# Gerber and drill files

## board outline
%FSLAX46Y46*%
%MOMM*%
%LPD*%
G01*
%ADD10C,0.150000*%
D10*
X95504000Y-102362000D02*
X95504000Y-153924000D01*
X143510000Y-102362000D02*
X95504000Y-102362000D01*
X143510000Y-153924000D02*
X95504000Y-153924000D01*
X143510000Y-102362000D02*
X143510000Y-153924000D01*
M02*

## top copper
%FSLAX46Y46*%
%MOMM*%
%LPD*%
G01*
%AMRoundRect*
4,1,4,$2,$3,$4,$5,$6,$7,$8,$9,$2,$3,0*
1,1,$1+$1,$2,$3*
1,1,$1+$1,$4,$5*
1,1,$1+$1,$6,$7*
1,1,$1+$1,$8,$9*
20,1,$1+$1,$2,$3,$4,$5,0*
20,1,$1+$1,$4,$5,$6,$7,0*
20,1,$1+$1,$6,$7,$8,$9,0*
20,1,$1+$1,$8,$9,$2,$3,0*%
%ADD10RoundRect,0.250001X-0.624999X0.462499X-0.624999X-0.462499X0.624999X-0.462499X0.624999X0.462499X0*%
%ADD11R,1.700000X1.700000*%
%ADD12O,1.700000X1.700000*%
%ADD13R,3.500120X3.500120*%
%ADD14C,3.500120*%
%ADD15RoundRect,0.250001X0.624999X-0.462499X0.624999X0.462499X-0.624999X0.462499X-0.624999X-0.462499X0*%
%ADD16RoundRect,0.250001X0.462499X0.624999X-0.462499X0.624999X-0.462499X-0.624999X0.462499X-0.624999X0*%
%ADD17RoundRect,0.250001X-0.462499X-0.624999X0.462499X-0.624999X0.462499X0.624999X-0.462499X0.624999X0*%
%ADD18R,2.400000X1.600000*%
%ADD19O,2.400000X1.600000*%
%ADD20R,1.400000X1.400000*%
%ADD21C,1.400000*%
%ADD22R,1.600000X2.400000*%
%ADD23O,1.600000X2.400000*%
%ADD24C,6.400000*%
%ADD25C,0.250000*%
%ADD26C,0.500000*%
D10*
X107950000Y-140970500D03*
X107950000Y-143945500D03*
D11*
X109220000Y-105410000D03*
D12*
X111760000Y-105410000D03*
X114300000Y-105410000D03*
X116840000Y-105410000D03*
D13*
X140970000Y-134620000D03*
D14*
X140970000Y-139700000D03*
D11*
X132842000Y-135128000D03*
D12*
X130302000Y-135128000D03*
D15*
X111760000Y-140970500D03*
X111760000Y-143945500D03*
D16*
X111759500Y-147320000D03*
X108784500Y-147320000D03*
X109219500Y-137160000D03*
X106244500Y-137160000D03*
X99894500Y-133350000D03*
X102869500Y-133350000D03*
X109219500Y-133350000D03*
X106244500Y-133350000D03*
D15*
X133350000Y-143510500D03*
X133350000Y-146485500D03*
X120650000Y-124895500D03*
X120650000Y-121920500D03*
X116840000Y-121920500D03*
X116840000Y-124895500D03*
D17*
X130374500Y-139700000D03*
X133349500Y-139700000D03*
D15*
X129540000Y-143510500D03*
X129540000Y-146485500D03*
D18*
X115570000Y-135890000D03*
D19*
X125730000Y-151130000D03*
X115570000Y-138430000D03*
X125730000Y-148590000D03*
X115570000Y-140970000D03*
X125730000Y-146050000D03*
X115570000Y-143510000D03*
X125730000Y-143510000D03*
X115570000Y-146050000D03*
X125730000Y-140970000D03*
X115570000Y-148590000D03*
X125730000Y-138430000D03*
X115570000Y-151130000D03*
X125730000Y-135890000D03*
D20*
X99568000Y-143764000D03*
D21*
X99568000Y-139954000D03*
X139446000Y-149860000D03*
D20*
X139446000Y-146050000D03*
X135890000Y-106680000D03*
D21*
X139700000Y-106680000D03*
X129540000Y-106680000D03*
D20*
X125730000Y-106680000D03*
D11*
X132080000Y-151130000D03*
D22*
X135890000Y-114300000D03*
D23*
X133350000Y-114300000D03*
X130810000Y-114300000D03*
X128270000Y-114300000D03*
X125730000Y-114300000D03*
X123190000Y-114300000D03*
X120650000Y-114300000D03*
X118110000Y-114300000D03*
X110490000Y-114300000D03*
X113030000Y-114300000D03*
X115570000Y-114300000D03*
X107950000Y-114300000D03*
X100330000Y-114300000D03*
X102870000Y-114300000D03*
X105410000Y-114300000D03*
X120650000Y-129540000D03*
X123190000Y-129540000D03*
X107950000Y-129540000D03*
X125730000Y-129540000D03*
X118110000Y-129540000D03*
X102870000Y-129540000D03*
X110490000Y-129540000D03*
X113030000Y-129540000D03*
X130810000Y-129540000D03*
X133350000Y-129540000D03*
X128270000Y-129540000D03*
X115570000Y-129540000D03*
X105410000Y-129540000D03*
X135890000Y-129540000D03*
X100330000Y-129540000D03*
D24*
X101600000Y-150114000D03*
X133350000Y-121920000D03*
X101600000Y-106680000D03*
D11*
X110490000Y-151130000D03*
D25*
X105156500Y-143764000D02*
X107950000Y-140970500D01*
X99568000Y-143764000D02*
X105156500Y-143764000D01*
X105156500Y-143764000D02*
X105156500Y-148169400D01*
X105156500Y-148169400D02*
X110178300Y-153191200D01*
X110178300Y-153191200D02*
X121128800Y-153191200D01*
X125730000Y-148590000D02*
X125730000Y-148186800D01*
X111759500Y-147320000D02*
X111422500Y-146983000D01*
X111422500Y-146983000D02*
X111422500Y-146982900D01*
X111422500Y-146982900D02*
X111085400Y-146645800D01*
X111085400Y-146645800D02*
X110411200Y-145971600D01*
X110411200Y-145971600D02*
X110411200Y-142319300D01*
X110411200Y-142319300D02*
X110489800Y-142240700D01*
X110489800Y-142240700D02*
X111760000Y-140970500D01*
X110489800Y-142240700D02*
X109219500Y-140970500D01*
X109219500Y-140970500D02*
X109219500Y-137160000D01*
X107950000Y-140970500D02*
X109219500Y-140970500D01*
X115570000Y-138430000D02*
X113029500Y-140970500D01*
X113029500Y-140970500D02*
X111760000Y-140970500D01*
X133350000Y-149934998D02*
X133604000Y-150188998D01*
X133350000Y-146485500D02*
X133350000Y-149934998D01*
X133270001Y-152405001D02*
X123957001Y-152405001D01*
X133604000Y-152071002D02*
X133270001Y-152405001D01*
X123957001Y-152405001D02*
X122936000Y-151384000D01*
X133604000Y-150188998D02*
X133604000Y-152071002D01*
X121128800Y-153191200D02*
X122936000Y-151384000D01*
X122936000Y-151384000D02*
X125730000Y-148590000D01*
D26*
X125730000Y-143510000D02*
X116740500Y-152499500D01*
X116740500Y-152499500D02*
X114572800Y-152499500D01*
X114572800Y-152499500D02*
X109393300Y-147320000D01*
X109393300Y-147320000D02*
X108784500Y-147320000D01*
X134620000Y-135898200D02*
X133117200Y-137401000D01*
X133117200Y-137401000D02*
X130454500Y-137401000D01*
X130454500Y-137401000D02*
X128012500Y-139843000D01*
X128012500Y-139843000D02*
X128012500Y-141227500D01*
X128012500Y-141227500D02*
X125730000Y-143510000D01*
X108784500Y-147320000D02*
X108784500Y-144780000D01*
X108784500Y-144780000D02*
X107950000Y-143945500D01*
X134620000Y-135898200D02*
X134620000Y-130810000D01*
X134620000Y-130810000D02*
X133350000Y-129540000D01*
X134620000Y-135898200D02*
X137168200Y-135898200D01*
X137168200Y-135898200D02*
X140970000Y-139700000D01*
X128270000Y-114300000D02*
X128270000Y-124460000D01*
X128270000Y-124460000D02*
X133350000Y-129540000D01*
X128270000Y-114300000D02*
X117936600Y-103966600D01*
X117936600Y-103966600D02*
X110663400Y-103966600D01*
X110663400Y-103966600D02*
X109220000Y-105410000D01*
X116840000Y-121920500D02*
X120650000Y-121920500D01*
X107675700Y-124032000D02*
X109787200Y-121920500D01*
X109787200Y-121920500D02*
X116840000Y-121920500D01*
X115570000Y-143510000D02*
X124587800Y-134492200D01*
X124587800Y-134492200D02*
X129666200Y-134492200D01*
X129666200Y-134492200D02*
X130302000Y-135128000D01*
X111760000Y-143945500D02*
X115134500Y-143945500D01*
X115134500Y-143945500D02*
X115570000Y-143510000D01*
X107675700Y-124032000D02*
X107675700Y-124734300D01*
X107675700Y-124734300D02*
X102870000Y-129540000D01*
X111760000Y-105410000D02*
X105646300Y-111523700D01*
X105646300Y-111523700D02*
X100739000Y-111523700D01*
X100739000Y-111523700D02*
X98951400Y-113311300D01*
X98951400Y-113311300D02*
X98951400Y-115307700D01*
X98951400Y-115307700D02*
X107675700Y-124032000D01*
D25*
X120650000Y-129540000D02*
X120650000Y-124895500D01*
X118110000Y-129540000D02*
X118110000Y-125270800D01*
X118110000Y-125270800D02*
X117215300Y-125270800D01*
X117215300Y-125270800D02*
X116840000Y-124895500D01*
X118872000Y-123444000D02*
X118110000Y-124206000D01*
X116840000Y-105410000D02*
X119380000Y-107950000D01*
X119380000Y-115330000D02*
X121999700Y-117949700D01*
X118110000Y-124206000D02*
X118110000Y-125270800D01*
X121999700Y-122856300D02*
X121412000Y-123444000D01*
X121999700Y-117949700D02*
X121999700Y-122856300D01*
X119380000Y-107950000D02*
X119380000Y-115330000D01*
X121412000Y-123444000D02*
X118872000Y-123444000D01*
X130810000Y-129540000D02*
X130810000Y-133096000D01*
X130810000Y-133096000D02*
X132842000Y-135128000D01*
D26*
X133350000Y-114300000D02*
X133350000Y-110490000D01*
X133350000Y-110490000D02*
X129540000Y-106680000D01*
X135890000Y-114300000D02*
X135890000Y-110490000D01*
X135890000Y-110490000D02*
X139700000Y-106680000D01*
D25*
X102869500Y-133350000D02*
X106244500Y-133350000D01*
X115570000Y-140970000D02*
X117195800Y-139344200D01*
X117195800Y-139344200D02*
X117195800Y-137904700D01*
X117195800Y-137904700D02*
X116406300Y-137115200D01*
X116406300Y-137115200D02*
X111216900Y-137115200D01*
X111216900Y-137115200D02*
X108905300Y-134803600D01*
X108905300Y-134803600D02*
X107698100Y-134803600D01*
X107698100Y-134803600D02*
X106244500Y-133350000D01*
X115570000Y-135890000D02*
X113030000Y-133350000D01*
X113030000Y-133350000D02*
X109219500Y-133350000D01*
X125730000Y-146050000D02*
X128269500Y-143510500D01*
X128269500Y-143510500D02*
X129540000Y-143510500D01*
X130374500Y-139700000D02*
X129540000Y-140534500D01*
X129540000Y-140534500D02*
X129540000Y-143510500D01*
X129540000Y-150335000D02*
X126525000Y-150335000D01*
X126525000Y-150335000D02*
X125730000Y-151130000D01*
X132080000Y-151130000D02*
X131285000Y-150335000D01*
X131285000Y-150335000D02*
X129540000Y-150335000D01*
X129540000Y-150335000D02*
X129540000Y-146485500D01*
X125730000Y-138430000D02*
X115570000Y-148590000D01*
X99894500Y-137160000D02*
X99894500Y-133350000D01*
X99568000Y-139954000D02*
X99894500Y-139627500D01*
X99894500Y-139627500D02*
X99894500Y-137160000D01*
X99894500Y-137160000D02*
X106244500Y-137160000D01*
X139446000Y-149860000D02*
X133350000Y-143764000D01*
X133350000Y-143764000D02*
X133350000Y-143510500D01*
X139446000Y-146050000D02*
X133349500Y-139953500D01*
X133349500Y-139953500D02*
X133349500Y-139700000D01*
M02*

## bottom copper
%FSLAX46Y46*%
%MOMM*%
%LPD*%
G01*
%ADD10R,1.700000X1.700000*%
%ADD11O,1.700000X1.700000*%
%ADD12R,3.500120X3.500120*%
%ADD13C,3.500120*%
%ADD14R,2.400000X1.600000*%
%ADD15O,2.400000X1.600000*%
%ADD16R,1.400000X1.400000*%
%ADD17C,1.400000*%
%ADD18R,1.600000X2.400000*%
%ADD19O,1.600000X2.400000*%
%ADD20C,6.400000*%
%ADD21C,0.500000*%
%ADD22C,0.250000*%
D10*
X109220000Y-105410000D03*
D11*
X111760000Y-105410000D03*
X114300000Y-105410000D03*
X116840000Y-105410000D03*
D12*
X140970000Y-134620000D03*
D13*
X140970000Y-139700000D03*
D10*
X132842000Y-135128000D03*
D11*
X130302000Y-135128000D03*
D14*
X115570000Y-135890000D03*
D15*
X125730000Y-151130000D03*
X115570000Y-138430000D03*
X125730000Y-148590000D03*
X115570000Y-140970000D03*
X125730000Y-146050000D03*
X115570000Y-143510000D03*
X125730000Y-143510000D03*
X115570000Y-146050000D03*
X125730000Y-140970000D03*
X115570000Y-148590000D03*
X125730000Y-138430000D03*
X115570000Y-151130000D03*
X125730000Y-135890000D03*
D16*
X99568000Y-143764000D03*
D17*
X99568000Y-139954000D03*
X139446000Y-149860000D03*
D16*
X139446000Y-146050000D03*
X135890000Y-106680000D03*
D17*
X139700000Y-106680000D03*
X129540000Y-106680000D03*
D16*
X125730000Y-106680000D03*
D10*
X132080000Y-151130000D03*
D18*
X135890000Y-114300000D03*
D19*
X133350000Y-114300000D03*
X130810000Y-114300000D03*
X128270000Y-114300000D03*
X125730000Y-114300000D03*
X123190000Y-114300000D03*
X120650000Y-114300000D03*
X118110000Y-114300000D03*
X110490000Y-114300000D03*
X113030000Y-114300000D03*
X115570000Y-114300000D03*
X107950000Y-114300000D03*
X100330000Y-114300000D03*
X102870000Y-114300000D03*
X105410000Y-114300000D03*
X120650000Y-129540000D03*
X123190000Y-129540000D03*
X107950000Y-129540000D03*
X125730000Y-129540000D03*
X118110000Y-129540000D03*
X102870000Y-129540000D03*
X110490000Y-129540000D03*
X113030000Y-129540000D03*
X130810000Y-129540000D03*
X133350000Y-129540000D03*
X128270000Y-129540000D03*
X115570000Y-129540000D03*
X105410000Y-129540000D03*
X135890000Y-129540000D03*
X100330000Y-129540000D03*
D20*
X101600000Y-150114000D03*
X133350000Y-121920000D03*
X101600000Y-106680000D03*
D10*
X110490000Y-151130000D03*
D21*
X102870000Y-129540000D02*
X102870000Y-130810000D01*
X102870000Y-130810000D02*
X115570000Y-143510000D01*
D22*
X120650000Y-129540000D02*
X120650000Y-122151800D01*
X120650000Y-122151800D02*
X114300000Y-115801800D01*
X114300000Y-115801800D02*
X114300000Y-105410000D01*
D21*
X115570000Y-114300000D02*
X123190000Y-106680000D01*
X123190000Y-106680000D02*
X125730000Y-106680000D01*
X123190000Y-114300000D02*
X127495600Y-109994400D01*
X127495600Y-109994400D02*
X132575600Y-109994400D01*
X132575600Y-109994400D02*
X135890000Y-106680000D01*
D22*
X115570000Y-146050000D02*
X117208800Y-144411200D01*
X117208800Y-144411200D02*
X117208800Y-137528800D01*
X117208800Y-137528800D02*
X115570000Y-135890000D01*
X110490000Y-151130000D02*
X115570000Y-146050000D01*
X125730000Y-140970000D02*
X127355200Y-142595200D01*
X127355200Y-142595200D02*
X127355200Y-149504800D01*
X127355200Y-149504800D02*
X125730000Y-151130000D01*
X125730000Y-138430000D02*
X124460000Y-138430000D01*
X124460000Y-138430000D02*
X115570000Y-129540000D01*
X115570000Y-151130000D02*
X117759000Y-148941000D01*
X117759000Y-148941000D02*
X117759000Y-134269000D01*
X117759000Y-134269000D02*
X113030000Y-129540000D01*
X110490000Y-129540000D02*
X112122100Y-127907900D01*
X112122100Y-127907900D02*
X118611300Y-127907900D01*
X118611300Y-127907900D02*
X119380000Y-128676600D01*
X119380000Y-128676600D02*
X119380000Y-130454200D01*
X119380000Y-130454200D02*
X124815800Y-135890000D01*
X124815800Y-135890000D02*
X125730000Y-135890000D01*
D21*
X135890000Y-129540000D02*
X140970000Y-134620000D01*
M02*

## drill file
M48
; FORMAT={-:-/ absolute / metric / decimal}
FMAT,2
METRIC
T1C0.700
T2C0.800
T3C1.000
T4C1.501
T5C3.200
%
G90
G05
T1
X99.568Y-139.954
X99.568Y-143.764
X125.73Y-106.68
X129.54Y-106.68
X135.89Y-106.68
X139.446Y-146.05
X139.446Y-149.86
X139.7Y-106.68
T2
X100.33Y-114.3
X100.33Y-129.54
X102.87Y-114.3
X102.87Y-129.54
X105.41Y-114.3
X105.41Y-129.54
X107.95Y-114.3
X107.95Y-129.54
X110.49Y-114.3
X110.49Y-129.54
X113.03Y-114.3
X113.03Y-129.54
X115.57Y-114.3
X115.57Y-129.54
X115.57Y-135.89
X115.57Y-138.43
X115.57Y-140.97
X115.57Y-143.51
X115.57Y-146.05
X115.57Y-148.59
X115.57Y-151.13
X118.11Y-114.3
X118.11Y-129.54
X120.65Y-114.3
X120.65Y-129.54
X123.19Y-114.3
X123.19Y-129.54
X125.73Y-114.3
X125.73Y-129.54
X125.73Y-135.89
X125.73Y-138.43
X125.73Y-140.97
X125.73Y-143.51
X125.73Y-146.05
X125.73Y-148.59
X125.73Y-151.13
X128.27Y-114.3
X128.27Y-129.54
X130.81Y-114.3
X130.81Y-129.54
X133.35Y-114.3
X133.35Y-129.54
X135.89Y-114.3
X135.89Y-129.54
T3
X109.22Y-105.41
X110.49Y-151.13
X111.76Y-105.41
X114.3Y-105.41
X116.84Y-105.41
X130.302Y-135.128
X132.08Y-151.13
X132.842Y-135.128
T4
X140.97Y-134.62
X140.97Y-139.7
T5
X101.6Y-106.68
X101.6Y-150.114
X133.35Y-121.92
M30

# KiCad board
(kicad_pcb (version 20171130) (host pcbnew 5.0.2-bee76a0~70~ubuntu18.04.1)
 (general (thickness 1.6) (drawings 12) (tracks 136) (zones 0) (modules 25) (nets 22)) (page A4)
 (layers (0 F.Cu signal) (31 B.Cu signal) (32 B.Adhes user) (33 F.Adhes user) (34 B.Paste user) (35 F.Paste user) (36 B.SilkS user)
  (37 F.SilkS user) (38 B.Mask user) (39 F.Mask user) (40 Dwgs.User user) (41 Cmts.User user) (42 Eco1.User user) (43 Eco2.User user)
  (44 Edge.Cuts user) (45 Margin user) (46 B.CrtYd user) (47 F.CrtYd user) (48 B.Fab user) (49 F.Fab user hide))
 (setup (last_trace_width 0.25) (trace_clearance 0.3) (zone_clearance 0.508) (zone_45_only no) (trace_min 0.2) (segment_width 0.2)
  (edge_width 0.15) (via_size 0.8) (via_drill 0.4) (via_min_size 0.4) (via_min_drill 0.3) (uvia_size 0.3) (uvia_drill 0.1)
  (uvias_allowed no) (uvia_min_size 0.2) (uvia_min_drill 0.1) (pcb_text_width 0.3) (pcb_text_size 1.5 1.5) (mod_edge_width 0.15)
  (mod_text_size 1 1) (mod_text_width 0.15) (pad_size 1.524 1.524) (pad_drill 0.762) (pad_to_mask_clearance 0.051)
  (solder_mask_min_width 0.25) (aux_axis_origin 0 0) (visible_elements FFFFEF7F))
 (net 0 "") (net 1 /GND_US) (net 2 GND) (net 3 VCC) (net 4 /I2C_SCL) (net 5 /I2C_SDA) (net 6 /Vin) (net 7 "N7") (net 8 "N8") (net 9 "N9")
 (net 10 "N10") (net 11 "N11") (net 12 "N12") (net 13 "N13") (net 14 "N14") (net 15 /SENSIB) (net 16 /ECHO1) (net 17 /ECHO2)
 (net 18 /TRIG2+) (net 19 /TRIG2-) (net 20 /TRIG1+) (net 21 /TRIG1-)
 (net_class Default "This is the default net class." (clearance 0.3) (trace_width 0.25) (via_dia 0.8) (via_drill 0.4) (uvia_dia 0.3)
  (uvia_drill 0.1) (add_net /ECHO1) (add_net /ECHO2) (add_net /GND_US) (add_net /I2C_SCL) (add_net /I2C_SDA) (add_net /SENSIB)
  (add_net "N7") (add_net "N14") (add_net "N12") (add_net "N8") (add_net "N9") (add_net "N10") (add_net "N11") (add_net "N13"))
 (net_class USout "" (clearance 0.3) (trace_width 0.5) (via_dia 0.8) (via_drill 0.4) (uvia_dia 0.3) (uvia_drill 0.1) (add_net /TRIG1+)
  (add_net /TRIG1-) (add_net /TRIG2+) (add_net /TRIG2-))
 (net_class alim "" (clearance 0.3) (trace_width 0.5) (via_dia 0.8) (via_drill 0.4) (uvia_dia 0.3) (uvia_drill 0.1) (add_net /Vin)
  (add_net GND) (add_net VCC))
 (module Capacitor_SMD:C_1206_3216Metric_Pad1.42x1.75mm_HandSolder (layer F.Cu) (at 107.95 142.458 270)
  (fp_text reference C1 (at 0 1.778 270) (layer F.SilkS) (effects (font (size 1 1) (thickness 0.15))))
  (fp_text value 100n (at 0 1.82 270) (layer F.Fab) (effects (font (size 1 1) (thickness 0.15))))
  (pad 1 smd roundrect (at -1.4875 0 270) (size 1.425 1.75) (layers F.Cu F.Paste F.Mask) (roundrect_rratio 0.175439) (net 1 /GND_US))
  (pad 2 smd roundrect (at 1.4875 0 270) (size 1.425 1.75) (layers F.Cu F.Paste F.Mask) (roundrect_rratio 0.175439) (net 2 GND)))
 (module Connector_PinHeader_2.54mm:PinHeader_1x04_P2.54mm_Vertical (layer F.Cu) (at 109.22 105.41 90)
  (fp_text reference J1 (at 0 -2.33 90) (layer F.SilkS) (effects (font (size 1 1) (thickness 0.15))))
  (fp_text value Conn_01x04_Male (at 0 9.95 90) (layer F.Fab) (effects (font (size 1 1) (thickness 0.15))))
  (pad 1 thru_hole rect (at 0 0 90) (size 1.7 1.7) (drill 1) (layers *.Cu *.Mask) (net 2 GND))
  (pad 2 thru_hole oval (at 0 2.54 90) (size 1.7 1.7) (drill 1) (layers *.Cu *.Mask) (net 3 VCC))
  (pad 3 thru_hole oval (at 0 5.08 90) (size 1.7 1.7) (drill 1) (layers *.Cu *.Mask) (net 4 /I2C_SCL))
  (pad 4 thru_hole oval (at 0 7.62 90) (size 1.7 1.7) (drill 1) (layers *.Cu *.Mask) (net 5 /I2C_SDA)))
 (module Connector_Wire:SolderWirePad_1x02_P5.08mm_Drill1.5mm (layer F.Cu) (at 140.97 134.62 270)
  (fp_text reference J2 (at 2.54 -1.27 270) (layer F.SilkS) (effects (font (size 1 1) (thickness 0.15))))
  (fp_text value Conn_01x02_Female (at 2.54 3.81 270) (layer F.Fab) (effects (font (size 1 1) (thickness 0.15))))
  (pad 1 thru_hole rect (at 0 0 270) (size 3.50012 3.50012) (drill 1.50114) (layers *.Cu *.Mask) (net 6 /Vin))
  (pad 2 thru_hole circle (at 5.08 0 270) (size 3.50012 3.50012) (drill 1.50114) (layers *.Cu *.Mask) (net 2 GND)))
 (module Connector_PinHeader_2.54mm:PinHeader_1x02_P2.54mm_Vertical (layer F.Cu) (at 132.842 135.128 270)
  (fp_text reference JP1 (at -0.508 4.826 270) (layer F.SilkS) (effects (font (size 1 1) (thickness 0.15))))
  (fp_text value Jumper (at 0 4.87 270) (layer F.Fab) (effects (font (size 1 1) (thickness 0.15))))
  (pad 1 thru_hole rect (at 0 0 270) (size 1.7 1.7) (drill 1) (layers *.Cu *.Mask) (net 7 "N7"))
  (pad 2 thru_hole oval (at 0 2.54 270) (size 1.7 1.7) (drill 1) (layers *.Cu *.Mask) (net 3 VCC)))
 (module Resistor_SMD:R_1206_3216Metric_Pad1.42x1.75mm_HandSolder (layer F.Cu) (at 111.76 142.458 90)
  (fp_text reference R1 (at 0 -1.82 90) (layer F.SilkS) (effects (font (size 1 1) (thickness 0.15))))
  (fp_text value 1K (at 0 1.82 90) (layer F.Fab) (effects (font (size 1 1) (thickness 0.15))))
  (pad 2 smd roundrect (at 1.4875 0 90) (size 1.425 1.75) (layers F.Cu F.Paste F.Mask) (roundrect_rratio 0.175439) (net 1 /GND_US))
  (pad 1 smd roundrect (at -1.4875 0 90) (size 1.425 1.75) (layers F.Cu F.Paste F.Mask) (roundrect_rratio 0.175439) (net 3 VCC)))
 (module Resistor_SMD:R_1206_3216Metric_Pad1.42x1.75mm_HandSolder (layer F.Cu) (at 110.272 147.32 180)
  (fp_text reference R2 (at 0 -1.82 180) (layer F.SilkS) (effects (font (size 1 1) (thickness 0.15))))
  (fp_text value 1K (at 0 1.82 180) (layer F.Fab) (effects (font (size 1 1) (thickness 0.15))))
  (pad 1 smd roundrect (at -1.4875 0 180) (size 1.425 1.75) (layers F.Cu F.Paste F.Mask) (roundrect_rratio 0.175439) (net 1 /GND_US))
  (pad 2 smd roundrect (at 1.4875 0 180) (size 1.425 1.75) (layers F.Cu F.Paste F.Mask) (roundrect_rratio 0.175439) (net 2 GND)))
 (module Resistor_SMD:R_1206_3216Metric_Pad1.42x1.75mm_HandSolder (layer F.Cu) (at 107.732 137.16 180)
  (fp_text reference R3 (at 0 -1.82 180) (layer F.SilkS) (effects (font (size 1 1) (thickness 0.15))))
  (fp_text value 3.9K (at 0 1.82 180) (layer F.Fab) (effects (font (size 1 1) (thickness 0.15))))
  (pad 1 smd roundrect (at -1.4875 0 180) (size 1.425 1.75) (layers F.Cu F.Paste F.Mask) (roundrect_rratio 0.175439) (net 1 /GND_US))
  (pad 2 smd roundrect (at 1.4875 0 180) (size 1.425 1.75) (layers F.Cu F.Paste F.Mask) (roundrect_rratio 0.175439) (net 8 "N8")))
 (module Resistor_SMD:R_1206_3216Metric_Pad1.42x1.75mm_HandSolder (layer F.Cu) (at 101.382 133.35 180)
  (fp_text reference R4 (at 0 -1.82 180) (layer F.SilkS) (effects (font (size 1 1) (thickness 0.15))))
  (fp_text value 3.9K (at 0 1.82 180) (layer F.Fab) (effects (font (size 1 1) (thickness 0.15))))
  (pad 2 smd roundrect (at 1.4875 0 180) (size 1.425 1.75) (layers F.Cu F.Paste F.Mask) (roundrect_rratio 0.175439) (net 8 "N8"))
  (pad 1 smd roundrect (at -1.4875 0 180) (size 1.425 1.75) (layers F.Cu F.Paste F.Mask) (roundrect_rratio 0.175439) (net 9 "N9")))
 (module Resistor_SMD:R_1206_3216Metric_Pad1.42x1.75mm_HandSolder (layer F.Cu) (at 107.732 133.35 180)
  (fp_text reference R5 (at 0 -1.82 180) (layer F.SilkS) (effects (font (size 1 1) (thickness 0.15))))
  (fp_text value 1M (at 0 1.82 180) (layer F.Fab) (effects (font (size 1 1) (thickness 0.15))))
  (pad 1 smd roundrect (at -1.4875 0 180) (size 1.425 1.75) (layers F.Cu F.Paste F.Mask) (roundrect_rratio 0.175439) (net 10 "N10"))
  (pad 2 smd roundrect (at 1.4875 0 180) (size 1.425 1.75) (layers F.Cu F.Paste F.Mask) (roundrect_rratio 0.175439) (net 9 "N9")))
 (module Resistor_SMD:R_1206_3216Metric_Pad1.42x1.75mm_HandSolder (layer F.Cu) (at 133.35 144.998 90)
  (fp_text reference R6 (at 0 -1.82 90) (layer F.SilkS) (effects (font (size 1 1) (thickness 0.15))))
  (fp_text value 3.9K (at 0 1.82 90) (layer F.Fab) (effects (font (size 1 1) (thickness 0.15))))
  (pad 2 smd roundrect (at 1.4875 0 90) (size 1.425 1.75) (layers F.Cu F.Paste F.Mask) (roundrect_rratio 0.175439) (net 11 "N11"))
  (pad 1 smd roundrect (at -1.4875 0 90) (size 1.425 1.75) (layers F.Cu F.Paste F.Mask) (roundrect_rratio 0.175439) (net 1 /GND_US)))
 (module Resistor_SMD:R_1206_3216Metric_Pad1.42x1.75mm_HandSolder (layer F.Cu) (at 120.65 123.408 90)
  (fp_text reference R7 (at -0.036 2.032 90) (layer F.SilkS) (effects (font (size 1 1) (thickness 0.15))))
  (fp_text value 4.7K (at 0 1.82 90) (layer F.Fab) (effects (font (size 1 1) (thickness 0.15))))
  (pad 1 smd roundrect (at -1.4875 0 90) (size 1.425 1.75) (layers F.Cu F.Paste F.Mask) (roundrect_rratio 0.175439) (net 4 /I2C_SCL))
  (pad 2 smd roundrect (at 1.4875 0 90) (size 1.425 1.75) (layers F.Cu F.Paste F.Mask) (roundrect_rratio 0.175439) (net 3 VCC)))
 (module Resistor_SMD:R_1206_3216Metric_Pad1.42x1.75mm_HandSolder (layer F.Cu) (at 116.84 123.408 90)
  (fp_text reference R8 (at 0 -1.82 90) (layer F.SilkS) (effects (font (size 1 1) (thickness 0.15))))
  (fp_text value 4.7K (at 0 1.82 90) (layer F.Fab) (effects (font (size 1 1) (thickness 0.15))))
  (pad 2 smd roundrect (at 1.4875 0 90) (size 1.425 1.75) (layers F.Cu F.Paste F.Mask) (roundrect_rratio 0.175439) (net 3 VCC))
  (pad 1 smd roundrect (at -1.4875 0 90) (size 1.425 1.75) (layers F.Cu F.Paste F.Mask) (roundrect_rratio 0.175439) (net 5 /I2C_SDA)))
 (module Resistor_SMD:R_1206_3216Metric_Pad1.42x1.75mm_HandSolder (layer F.Cu) (at 131.862 139.7)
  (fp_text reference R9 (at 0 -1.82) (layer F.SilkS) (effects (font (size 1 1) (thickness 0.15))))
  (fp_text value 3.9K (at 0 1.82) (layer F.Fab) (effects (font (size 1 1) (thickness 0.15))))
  (pad 1 smd roundrect (at -1.4875 0) (size 1.425 1.75) (layers F.Cu F.Paste F.Mask) (roundrect_rratio 0.175439) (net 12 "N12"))
  (pad 2 smd roundrect (at 1.4875 0) (size 1.425 1.75) (layers F.Cu F.Paste F.Mask) (roundrect_rratio 0.175439) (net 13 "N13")))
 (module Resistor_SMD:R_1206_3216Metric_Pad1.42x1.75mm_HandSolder (layer F.Cu) (at 129.54 144.998 90)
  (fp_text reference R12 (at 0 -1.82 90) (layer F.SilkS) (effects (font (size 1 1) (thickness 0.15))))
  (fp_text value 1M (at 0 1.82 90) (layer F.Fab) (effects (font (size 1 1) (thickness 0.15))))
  (pad 2 smd roundrect (at 1.4875 0 90) (size 1.425 1.75) (layers F.Cu F.Paste F.Mask) (roundrect_rratio 0.175439) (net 12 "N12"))
  (pad 1 smd roundrect (at -1.4875 0 90) (size 1.425 1.75) (layers F.Cu F.Paste F.Mask) (roundrect_rratio 0.175439) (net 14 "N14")))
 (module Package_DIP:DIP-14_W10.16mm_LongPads (layer F.Cu) (at 115.57 135.89)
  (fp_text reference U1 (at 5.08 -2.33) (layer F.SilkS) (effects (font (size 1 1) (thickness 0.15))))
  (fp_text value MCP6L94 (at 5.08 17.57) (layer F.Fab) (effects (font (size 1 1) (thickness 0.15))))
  (pad 1 thru_hole rect (at 0 0) (size 2.4 1.6) (drill 0.8) (layers *.Cu *.Mask) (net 10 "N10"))
  (pad 8 thru_hole oval (at 10.16 15.24) (size 2.4 1.6) (drill 0.8) (layers *.Cu *.Mask) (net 14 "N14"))
  (pad 2 thru_hole oval (at 0 2.54) (size 2.4 1.6) (drill 0.8) (layers *.Cu *.Mask) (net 1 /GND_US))
  (pad 9 thru_hole oval (at 10.16 12.7) (size 2.4 1.6) (drill 0.8) (layers *.Cu *.Mask) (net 1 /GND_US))
  (pad 3 thru_hole oval (at 0 5.08) (size 2.4 1.6) (drill 0.8) (layers *.Cu *.Mask) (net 9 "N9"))
  (pad 10 thru_hole oval (at 10.16 10.16) (size 2.4 1.6) (drill 0.8) (layers *.Cu *.Mask) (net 12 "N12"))
  (pad 4 thru_hole oval (at 0 7.62) (size 2.4 1.6) (drill 0.8) (layers *.Cu *.Mask) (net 3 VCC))
  (pad 11 thru_hole oval (at 10.16 7.62) (size 2.4 1.6) (drill 0.8) (layers *.Cu *.Mask) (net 2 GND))
  (pad 5 thru_hole oval (at 0 10.16) (size 2.4 1.6) (drill 0.8) (layers *.Cu *.Mask) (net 10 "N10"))
  (pad 12 thru_hole oval (at 10.16 5.08) (size 2.4 1.6) (drill 0.8) (layers *.Cu *.Mask) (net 14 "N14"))
  (pad 6 thru_hole oval (at 0 12.7) (size 2.4 1.6) (drill 0.8) (layers *.Cu *.Mask) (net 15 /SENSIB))
  (pad 13 thru_hole oval (at 10.16 2.54) (size 2.4 1.6) (drill 0.8) (layers *.Cu *.Mask) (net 15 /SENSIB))
  (pad 7 thru_hole oval (at 0 15.24) (size 2.4 1.6) (drill 0.8) (layers *.Cu *.Mask) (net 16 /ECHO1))
  (pad 14 thru_hole oval (at 10.16 0) (size 2.4 1.6) (drill 0.8) (layers *.Cu *.Mask) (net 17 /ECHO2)))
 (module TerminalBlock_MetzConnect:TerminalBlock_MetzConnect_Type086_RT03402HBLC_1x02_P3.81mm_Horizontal (layer F.Cu) (at 99.568 143.764 90)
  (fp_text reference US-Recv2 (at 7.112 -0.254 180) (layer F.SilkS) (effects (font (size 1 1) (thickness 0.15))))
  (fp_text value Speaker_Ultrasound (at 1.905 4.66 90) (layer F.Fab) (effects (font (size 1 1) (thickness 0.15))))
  (pad 1 thru_hole rect (at 0 0 90) (size 1.4 1.4) (drill 0.7) (layers *.Cu *.Mask) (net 1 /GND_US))
  (pad 2 thru_hole circle (at 3.81 0 90) (size 1.4 1.4) (drill 0.7) (layers *.Cu *.Mask) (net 8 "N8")))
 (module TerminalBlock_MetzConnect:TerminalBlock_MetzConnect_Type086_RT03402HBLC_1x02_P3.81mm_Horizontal (layer F.Cu)
  (at 139.446 146.05 270)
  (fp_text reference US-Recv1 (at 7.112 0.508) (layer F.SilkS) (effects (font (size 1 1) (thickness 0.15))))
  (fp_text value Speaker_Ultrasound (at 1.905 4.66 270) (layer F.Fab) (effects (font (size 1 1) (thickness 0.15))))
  (pad 2 thru_hole circle (at 3.81 0 270) (size 1.4 1.4) (drill 0.7) (layers *.Cu *.Mask) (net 11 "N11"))
  (pad 1 thru_hole rect (at 0 0 270) (size 1.4 1.4) (drill 0.7) (layers *.Cu *.Mask) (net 13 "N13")))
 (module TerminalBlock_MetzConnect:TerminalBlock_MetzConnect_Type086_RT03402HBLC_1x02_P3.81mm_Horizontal (layer F.Cu) (at 135.89 106.68)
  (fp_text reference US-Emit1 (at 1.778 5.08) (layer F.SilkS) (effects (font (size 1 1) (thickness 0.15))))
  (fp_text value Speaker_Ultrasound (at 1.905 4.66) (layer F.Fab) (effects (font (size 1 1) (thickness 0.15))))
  (pad 1 thru_hole rect (at 0 0) (size 1.4 1.4) (drill 0.7) (layers *.Cu *.Mask) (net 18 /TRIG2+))
  (pad 2 thru_hole circle (at 3.81 0) (size 1.4 1.4) (drill 0.7) (layers *.Cu *.Mask) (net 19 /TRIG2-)))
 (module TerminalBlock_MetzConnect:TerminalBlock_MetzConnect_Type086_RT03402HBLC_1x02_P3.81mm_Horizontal (layer F.Cu) (at 125.73 106.68)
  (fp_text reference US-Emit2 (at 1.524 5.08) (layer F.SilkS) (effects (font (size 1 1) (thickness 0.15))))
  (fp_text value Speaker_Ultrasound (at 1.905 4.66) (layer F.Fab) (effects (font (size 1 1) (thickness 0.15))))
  (pad 2 thru_hole circle (at 3.81 0) (size 1.4 1.4) (drill 0.7) (layers *.Cu *.Mask) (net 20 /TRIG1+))
  (pad 1 thru_hole rect (at 0 0) (size 1.4 1.4) (drill 0.7) (layers *.Cu *.Mask) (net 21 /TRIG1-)))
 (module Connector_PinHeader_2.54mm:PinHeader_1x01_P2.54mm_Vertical (layer F.Cu) (at 132.08 151.13)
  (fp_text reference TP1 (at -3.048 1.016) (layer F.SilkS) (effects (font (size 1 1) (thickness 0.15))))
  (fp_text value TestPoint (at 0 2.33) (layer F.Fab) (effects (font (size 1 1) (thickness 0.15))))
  (pad 1 thru_hole rect (at 0 0) (size 1.7 1.7) (drill 1) (layers *.Cu *.Mask) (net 14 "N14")))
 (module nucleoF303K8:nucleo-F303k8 (layer F.Cu) (at 135.89 121.92 270)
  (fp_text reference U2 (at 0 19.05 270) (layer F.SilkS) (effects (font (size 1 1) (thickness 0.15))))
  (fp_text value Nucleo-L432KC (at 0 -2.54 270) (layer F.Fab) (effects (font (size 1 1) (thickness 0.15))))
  (pad 1 thru_hole rect (at -7.62 0 270) (size 2.4 1.6) (drill 0.8) (layers *.Cu *.Mask) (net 19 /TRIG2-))
  (pad 2 thru_hole oval (at -7.62 2.54 270) (size 2.4 1.6) (drill 0.8) (layers *.Cu *.Mask) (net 20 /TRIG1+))
  (pad 3 thru_hole oval (at -7.62 5.08 270) (size 2.4 1.6) (drill 0.8) (layers *.Cu *.Mask))
  (pad 4 thru_hole oval (at -7.62 7.62 270) (size 2.4 1.6) (drill 0.8) (layers *.Cu *.Mask) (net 2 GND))
  (pad 5 thru_hole oval (at -7.62 10.16 270) (size 2.4 1.6) (drill 0.8) (layers *.Cu *.Mask))
  (pad 6 thru_hole oval (at -7.62 12.7 270) (size 2.4 1.6) (drill 0.8) (layers *.Cu *.Mask) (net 18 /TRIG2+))
  (pad 7 thru_hole oval (at -7.62 15.24 270) (size 2.4 1.6) (drill 0.8) (layers *.Cu *.Mask))
  (pad 8 thru_hole oval (at -7.62 17.78 270) (size 2.4 1.6) (drill 0.8) (layers *.Cu *.Mask))
  (pad 11 thru_hole oval (at -7.62 25.4 270) (size 2.4 1.6) (drill 0.8) (layers *.Cu *.Mask))
  (pad 10 thru_hole oval (at -7.62 22.86 270) (size 2.4 1.6) (drill 0.8) (layers *.Cu *.Mask))
  (pad 9 thru_hole oval (at -7.62 20.32 270) (size 2.4 1.6) (drill 0.8) (layers *.Cu *.Mask) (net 21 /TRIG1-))
  (pad 12 thru_hole oval (at -7.62 27.94 270) (size 2.4 1.6) (drill 0.8) (layers *.Cu *.Mask))
  (pad 15 thru_hole oval (at -7.62 35.56 270) (size 2.4 1.6) (drill 0.8) (layers *.Cu *.Mask))
  (pad 14 thru_hole oval (at -7.62 33.02 270) (size 2.4 1.6) (drill 0.8) (layers *.Cu *.Mask))
  (pad 13 thru_hole oval (at -7.62 30.48 270) (size 2.4 1.6) (drill 0.8) (layers *.Cu *.Mask))
  (pad 24 thru_hole oval (at 7.62 15.24 270) (size 2.4 1.6) (drill 0.8) (layers *.Cu *.Mask) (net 4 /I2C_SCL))
  (pad 25 thru_hole oval (at 7.62 12.7 270) (size 2.4 1.6) (drill 0.8) (layers *.Cu *.Mask))
  (pad 19 thru_hole oval (at 7.62 27.94 270) (size 2.4 1.6) (drill 0.8) (layers *.Cu *.Mask))
  (pad 26 thru_hole oval (at 7.62 10.16 270) (size 2.4 1.6) (drill 0.8) (layers *.Cu *.Mask))
  (pad 23 thru_hole oval (at 7.62 17.78 270) (size 2.4 1.6) (drill 0.8) (layers *.Cu *.Mask) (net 5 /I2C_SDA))
  (pad 17 thru_hole oval (at 7.62 33.02 270) (size 2.4 1.6) (drill 0.8) (layers *.Cu *.Mask) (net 3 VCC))
  (pad 20 thru_hole oval (at 7.62 25.4 270) (size 2.4 1.6) (drill 0.8) (layers *.Cu *.Mask) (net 17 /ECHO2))
  (pad 21 thru_hole oval (at 7.62 22.86 270) (size 2.4 1.6) (drill 0.8) (layers *.Cu *.Mask) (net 16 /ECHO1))
  (pad 28 thru_hole oval (at 7.62 5.08 270) (size 2.4 1.6) (drill 0.8) (layers *.Cu *.Mask) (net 7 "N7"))
  (pad 29 thru_hole oval (at 7.62 2.54 270) (size 2.4 1.6) (drill 0.8) (layers *.Cu *.Mask) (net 2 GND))
  (pad 27 thru_hole oval (at 7.62 7.62 270) (size 2.4 1.6) (drill 0.8) (layers *.Cu *.Mask))
  (pad 22 thru_hole oval (at 7.62 20.32 270) (size 2.4 1.6) (drill 0.8) (layers *.Cu *.Mask) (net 15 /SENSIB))
  (pad 18 thru_hole oval (at 7.62 30.48 270) (size 2.4 1.6) (drill 0.8) (layers *.Cu *.Mask))
  (pad 30 thru_hole oval (at 7.62 0 270) (size 2.4 1.6) (drill 0.8) (layers *.Cu *.Mask) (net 6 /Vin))
  (pad 16 thru_hole oval (at 7.62 35.56 270) (size 2.4 1.6) (drill 0.8) (layers *.Cu *.Mask)))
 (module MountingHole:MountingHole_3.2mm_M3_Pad (layer F.Cu) (at 101.6 150.114)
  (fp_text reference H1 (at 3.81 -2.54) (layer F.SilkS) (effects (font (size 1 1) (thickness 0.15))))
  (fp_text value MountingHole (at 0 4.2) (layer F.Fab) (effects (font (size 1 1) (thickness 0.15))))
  (pad 1 thru_hole circle (at 0 0) (size 6.4 6.4) (drill 3.2) (layers *.Cu *.Mask)))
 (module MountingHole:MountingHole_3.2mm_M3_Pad (layer F.Cu) (at 133.35 121.92)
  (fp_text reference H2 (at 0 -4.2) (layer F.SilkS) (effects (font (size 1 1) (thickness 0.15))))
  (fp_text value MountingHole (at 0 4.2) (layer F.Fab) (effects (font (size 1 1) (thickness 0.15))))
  (pad 1 thru_hole circle (at 0 0) (size 6.4 6.4) (drill 3.2) (layers *.Cu *.Mask)))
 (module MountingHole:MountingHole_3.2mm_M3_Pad (layer F.Cu) (at 101.6 106.68)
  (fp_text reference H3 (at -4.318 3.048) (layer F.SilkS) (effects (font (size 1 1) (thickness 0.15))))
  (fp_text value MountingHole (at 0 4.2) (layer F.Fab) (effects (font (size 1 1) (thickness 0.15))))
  (pad 1 thru_hole circle (at 0 0) (size 6.4 6.4) (drill 3.2) (layers *.Cu *.Mask)))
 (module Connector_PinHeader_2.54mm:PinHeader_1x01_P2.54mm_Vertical (layer F.Cu) (at 110.49 151.13)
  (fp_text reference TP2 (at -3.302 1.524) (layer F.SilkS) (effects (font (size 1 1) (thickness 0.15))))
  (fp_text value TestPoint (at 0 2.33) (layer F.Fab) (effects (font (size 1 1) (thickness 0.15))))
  (pad 1 thru_hole rect (at 0 0) (size 1.7 1.7) (drill 1) (layers *.Cu *.Mask) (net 10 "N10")))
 (gr_line (start 95.504 102.362) (end 95.504 153.924) (layer Edge.Cuts) (width 0.15))
 (gr_line (start 143.51 102.362) (end 95.504 102.362) (layer Edge.Cuts) (width 0.15))
 (gr_line (start 143.51 153.924) (end 95.504 153.924) (layer Edge.Cuts) (width 0.15))
 (gr_line (start 143.51 102.362) (end 143.51 153.924) (layer Edge.Cuts) (width 0.15))
 (segment (start 105.1565 143.764) (end 107.95 140.9705) (width 0.25) (layer F.Cu) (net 1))
 (segment (start 99.568 143.764) (end 105.1565 143.764) (width 0.25) (layer F.Cu) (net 1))
 (segment (start 105.1565 143.764) (end 105.1565 148.1694) (width 0.25) (layer F.Cu) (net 1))
 (segment (start 105.1565 148.1694) (end 110.1783 153.1912) (width 0.25) (layer F.Cu) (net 1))
 (segment (start 110.1783 153.1912) (end 121.1288 153.1912) (width 0.25) (layer F.Cu) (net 1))
 (segment (start 125.73 148.59) (end 125.73 148.1868) (width 0.25) (layer F.Cu) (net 1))
 (segment (start 111.7595 147.32) (end 111.4225 146.983) (width 0.25) (layer F.Cu) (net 1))
 (segment (start 111.4225 146.983) (end 111.4225 146.9829) (width 0.25) (layer F.Cu) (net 1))
 (segment (start 111.4225 146.9829) (end 111.0854 146.6458) (width 0.25) (layer F.Cu) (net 1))
 (segment (start 111.0854 146.6458) (end 110.4112 145.9716) (width 0.25) (layer F.Cu) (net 1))
 (segment (start 110.4112 145.9716) (end 110.4112 142.3193) (width 0.25) (layer F.Cu) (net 1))
 (segment (start 110.4112 142.3193) (end 110.4898 142.2407) (width 0.25) (layer F.Cu) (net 1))
 (segment (start 110.4898 142.2407) (end 111.76 140.9705) (width 0.25) (layer F.Cu) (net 1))
 (segment (start 110.4898 142.2407) (end 109.2195 140.9705) (width 0.25) (layer F.Cu) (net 1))
 (segment (start 109.2195 140.9705) (end 109.2195 137.16) (width 0.25) (layer F.Cu) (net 1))
 (segment (start 107.95 140.9705) (end 109.2195 140.9705) (width 0.25) (layer F.Cu) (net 1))
 (segment (start 115.57 138.43) (end 113.0295 140.9705) (width 0.25) (layer F.Cu) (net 1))
 (segment (start 113.0295 140.9705) (end 111.76 140.9705) (width 0.25) (layer F.Cu) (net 1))
 (segment (start 133.35 149.934998) (end 133.604 150.188998) (width 0.25) (layer F.Cu) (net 1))
 (segment (start 133.35 146.4855) (end 133.35 149.934998) (width 0.25) (layer F.Cu) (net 1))
 (segment (start 133.270001 152.405001) (end 123.957001 152.405001) (width 0.25) (layer F.Cu) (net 1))
 (segment (start 133.604 152.071002) (end 133.270001 152.405001) (width 0.25) (layer F.Cu) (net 1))
 (segment (start 123.957001 152.405001) (end 122.936 151.384) (width 0.25) (layer F.Cu) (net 1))
 (segment (start 133.604 150.188998) (end 133.604 152.071002) (width 0.25) (layer F.Cu) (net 1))
 (segment (start 121.1288 153.1912) (end 122.936 151.384) (width 0.25) (layer F.Cu) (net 1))
 (segment (start 122.936 151.384) (end 125.73 148.59) (width 0.25) (layer F.Cu) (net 1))
 (segment (start 125.73 143.51) (end 116.7405 152.4995) (width 0.5) (layer F.Cu) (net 2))
 (segment (start 116.7405 152.4995) (end 114.5728 152.4995) (width 0.5) (layer F.Cu) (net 2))
 (segment (start 114.5728 152.4995) (end 109.3933 147.32) (width 0.5) (layer F.Cu) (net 2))
 (segment (start 109.3933 147.32) (end 108.7845 147.32) (width 0.5) (layer F.Cu) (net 2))
 (segment (start 134.62 135.8982) (end 133.1172 137.401) (width 0.5) (layer F.Cu) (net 2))
 (segment (start 133.1172 137.401) (end 130.4545 137.401) (width 0.5) (layer F.Cu) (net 2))
 (segment (start 130.4545 137.401) (end 128.0125 139.843) (width 0.5) (layer F.Cu) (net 2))
 (segment (start 128.0125 139.843) (end 128.0125 141.2275) (width 0.5) (layer F.Cu) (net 2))
 (segment (start 128.0125 141.2275) (end 125.73 143.51) (width 0.5) (layer F.Cu) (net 2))
 (segment (start 108.7845 147.32) (end 108.7845 144.78) (width 0.5) (layer F.Cu) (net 2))
 (segment (start 108.7845 144.78) (end 107.95 143.9455) (width 0.5) (layer F.Cu) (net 2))
 (segment (start 134.62 135.8982) (end 134.62 130.81) (width 0.5) (layer F.Cu) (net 2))
 (segment (start 134.62 130.81) (end 133.35 129.54) (width 0.5) (layer F.Cu) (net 2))
 (segment (start 134.62 135.8982) (end 137.1682 135.8982) (width 0.5) (layer F.Cu) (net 2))
 (segment (start 137.1682 135.8982) (end 140.97 139.7) (width 0.5) (layer F.Cu) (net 2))
 (segment (start 128.27 114.3) (end 128.27 124.46) (width 0.5) (layer F.Cu) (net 2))
 (segment (start 128.27 124.46) (end 133.35 129.54) (width 0.5) (layer F.Cu) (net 2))
 (segment (start 128.27 114.3) (end 117.9366 103.9666) (width 0.5) (layer F.Cu) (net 2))
 (segment (start 117.9366 103.9666) (end 110.6634 103.9666) (width 0.5) (layer F.Cu) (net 2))
 (segment (start 110.6634 103.9666) (end 109.22 105.41) (width 0.5) (layer F.Cu) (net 2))
 (segment (start 116.84 121.9205) (end 120.65 121.9205) (width 0.5) (layer F.Cu) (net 3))
 (segment (start 107.6757 124.032) (end 109.7872 121.9205) (width 0.5) (layer F.Cu) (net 3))
 (segment (start 109.7872 121.9205) (end 116.84 121.9205) (width 0.5) (layer F.Cu) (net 3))
 (segment (start 115.57 143.51) (end 124.5878 134.4922) (width 0.5) (layer F.Cu) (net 3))
 (segment (start 124.5878 134.4922) (end 129.6662 134.4922) (width 0.5) (layer F.Cu) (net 3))
 (segment (start 129.6662 134.4922) (end 130.302 135.128) (width 0.5) (layer F.Cu) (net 3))
 (segment (start 111.76 143.9455) (end 115.1345 143.9455) (width 0.5) (layer F.Cu) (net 3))
 (segment (start 115.1345 143.9455) (end 115.57 143.51) (width 0.5) (layer F.Cu) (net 3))
 (segment (start 102.87 129.54) (end 102.87 130.81) (width 0.5) (layer B.Cu) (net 3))
 (segment (start 102.87 130.81) (end 115.57 143.51) (width 0.5) (layer B.Cu) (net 3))
 (segment (start 107.6757 124.032) (end 107.6757 124.7343) (width 0.5) (layer F.Cu) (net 3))
 (segment (start 107.6757 124.7343) (end 102.87 129.54) (width 0.5) (layer F.Cu) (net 3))
 (segment (start 111.76 105.41) (end 105.6463 111.5237) (width 0.5) (layer F.Cu) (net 3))
 (segment (start 105.6463 111.5237) (end 100.739 111.5237) (width 0.5) (layer F.Cu) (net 3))
 (segment (start 100.739 111.5237) (end 98.9514 113.3113) (width 0.5) (layer F.Cu) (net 3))
 (segment (start 98.9514 113.3113) (end 98.9514 115.3077) (width 0.5) (layer F.Cu) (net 3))
 (segment (start 98.9514 115.3077) (end 107.6757 124.032) (width 0.5) (layer F.Cu) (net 3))
 (segment (start 120.65 129.54) (end 120.65 124.8955) (width 0.25) (layer F.Cu) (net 4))
 (segment (start 120.65 129.54) (end 120.65 122.1518) (width 0.25) (layer B.Cu) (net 4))
 (segment (start 120.65 122.1518) (end 114.3 115.8018) (width 0.25) (layer B.Cu) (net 4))
 (segment (start 114.3 115.8018) (end 114.3 105.41) (width 0.25) (layer B.Cu) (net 4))
 (segment (start 118.11 129.54) (end 118.11 125.2708) (width 0.25) (layer F.Cu) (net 5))
 (segment (start 118.11 125.2708) (end 117.2153 125.2708) (width 0.25) (layer F.Cu) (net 5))
 (segment (start 117.2153 125.2708) (end 116.84 124.8955) (width 0.25) (layer F.Cu) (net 5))
 (segment (start 118.872 123.444) (end 118.11 124.206) (width 0.25) (layer F.Cu) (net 5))
 (segment (start 116.84 105.41) (end 119.38 107.95) (width 0.25) (layer F.Cu) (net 5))
 (segment (start 119.38 115.33) (end 121.9997 117.9497) (width 0.25) (layer F.Cu) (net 5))
 (segment (start 118.11 124.206) (end 118.11 125.2708) (width 0.25) (layer F.Cu) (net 5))
 (segment (start 121.9997 122.8563) (end 121.412 123.444) (width 0.25) (layer F.Cu) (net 5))
 (segment (start 121.9997 117.9497) (end 121.9997 122.8563) (width 0.25) (layer F.Cu) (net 5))
 (segment (start 119.38 107.95) (end 119.38 115.33) (width 0.25) (layer F.Cu) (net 5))
 (segment (start 121.412 123.444) (end 118.872 123.444) (width 0.25) (layer F.Cu) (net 5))
 (segment (start 130.81 129.54) (end 130.81 133.096) (width 0.25) (layer F.Cu) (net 7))
 (segment (start 130.81 133.096) (end 132.842 135.128) (width 0.25) (layer F.Cu) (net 7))
 (segment (start 115.57 114.3) (end 123.19 106.68) (width 0.5) (layer B.Cu) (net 21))
 (segment (start 123.19 106.68) (end 125.73 106.68) (width 0.5) (layer B.Cu) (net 21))
 (segment (start 133.35 114.3) (end 133.35 110.49) (width 0.5) (layer F.Cu) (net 20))
 (segment (start 133.35 110.49) (end 129.54 106.68) (width 0.5) (layer F.Cu) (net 20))
 (segment (start 123.19 114.3) (end 127.4956 109.9944) (width 0.5) (layer B.Cu) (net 18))
 (segment (start 127.4956 109.9944) (end 132.5756 109.9944) (width 0.5) (layer B.Cu) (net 18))
 (segment (start 132.5756 109.9944) (end 135.89 106.68) (width 0.5) (layer B.Cu) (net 18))
 (segment (start 135.89 114.3) (end 135.89 110.49) (width 0.5) (layer F.Cu) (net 19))
 (segment (start 135.89 110.49) (end 139.7 106.68) (width 0.5) (layer F.Cu) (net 19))
 (segment (start 102.8695 133.35) (end 106.2445 133.35) (width 0.25) (layer F.Cu) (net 9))
 (segment (start 115.57 140.97) (end 117.1958 139.3442) (width 0.25) (layer F.Cu) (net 9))
 (segment (start 117.1958 139.3442) (end 117.1958 137.9047) (width 0.25) (layer F.Cu) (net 9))
 (segment (start 117.1958 137.9047) (end 116.4063 137.1152) (width 0.25) (layer F.Cu) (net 9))
 (segment (start 116.4063 137.1152) (end 111.2169 137.1152) (width 0.25) (layer F.Cu) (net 9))
 (segment (start 111.2169 137.1152) (end 108.9053 134.8036) (width 0.25) (layer F.Cu) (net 9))
 (segment (start 108.9053 134.8036) (end 107.6981 134.8036) (width 0.25) (layer F.Cu) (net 9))
 (segment (start 107.6981 134.8036) (end 106.2445 133.35) (width 0.25) (layer F.Cu) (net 9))
 (segment (start 115.57 146.05) (end 117.2088 144.4112) (width 0.25) (layer B.Cu) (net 10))
 (segment (start 117.2088 144.4112) (end 117.2088 137.5288) (width 0.25) (layer B.Cu) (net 10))
 (segment (start 117.2088 137.5288) (end 115.57 135.89) (width 0.25) (layer B.Cu) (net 10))
 (segment (start 110.49 151.13) (end 115.57 146.05) (width 0.25) (layer B.Cu) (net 10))
 (segment (start 115.57 135.89) (end 113.03 133.35) (width 0.25) (layer F.Cu) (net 10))
 (segment (start 113.03 133.35) (end 109.2195 133.35) (width 0.25) (layer F.Cu) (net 10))
 (segment (start 125.73 146.05) (end 128.2695 143.5105) (width 0.25) (layer F.Cu) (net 12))
 (segment (start 128.2695 143.5105) (end 129.54 143.5105) (width 0.25) (layer F.Cu) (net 12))
 (segment (start 130.3745 139.7) (end 129.54 140.5345) (width 0.25) (layer F.Cu) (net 12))
 (segment (start 129.54 140.5345) (end 129.54 143.5105) (width 0.25) (layer F.Cu) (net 12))
 (segment (start 125.73 140.97) (end 127.3552 142.5952) (width 0.25) (layer B.Cu) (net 14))
 (segment (start 127.3552 142.5952) (end 127.3552 149.5048) (width 0.25) (layer B.Cu) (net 14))
 (segment (start 127.3552 149.5048) (end 125.73 151.13) (width 0.25) (layer B.Cu) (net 14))
 (segment (start 129.54 150.335) (end 126.525 150.335) (width 0.25) (layer F.Cu) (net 14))
 (segment (start 126.525 150.335) (end 125.73 151.13) (width 0.25) (layer F.Cu) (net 14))
 (segment (start 132.08 151.13) (end 131.285 150.335) (width 0.25) (layer F.Cu) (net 14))
 (segment (start 131.285 150.335) (end 129.54 150.335) (width 0.25) (layer F.Cu) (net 14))
 (segment (start 129.54 150.335) (end 129.54 146.4855) (width 0.25) (layer F.Cu) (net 14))
 (segment (start 125.73 138.43) (end 115.57 148.59) (width 0.25) (layer F.Cu) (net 15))
 (segment (start 125.73 138.43) (end 124.46 138.43) (width 0.25) (layer B.Cu) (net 15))
 (segment (start 124.46 138.43) (end 115.57 129.54) (width 0.25) (layer B.Cu) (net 15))
 (segment (start 115.57 151.13) (end 117.759 148.941) (width 0.25) (layer B.Cu) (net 16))
 (segment (start 117.759 148.941) (end 117.759 134.269) (width 0.25) (layer B.Cu) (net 16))
 (segment (start 117.759 134.269) (end 113.03 129.54) (width 0.25) (layer B.Cu) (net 16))
 (segment (start 110.49 129.54) (end 112.1221 127.9079) (width 0.25) (layer B.Cu) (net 17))
 (segment (start 112.1221 127.9079) (end 118.6113 127.9079) (width 0.25) (layer B.Cu) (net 17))
 (segment (start 118.6113 127.9079) (end 119.38 128.6766) (width 0.25) (layer B.Cu) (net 17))
 (segment (start 119.38 128.6766) (end 119.38 130.4542) (width 0.25) (layer B.Cu) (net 17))
 (segment (start 119.38 130.4542) (end 124.8158 135.89) (width 0.25) (layer B.Cu) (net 17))
 (segment (start 124.8158 135.89) (end 125.73 135.89) (width 0.25) (layer B.Cu) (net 17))
 (segment (start 135.89 129.54) (end 140.97 134.62) (width 0.5) (layer B.Cu) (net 6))
 (segment (start 99.8945 137.16) (end 99.8945 133.35) (width 0.25) (layer F.Cu) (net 8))
 (segment (start 99.568 139.954) (end 99.8945 139.6275) (width 0.25) (layer F.Cu) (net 8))
 (segment (start 99.8945 139.6275) (end 99.8945 137.16) (width 0.25) (layer F.Cu) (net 8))
 (segment (start 99.8945 137.16) (end 106.2445 137.16) (width 0.25) (layer F.Cu) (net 8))
 (segment (start 139.446 149.86) (end 133.35 143.764) (width 0.25) (layer F.Cu) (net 11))
 (segment (start 133.35 143.764) (end 133.35 143.5105) (width 0.25) (layer F.Cu) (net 11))
 (segment (start 139.446 146.05) (end 133.3495 139.9535) (width 0.25) (layer F.Cu) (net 13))
 (segment (start 133.3495 139.9535) (end 133.3495 139.7) (width 0.25) (layer F.Cu) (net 13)))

